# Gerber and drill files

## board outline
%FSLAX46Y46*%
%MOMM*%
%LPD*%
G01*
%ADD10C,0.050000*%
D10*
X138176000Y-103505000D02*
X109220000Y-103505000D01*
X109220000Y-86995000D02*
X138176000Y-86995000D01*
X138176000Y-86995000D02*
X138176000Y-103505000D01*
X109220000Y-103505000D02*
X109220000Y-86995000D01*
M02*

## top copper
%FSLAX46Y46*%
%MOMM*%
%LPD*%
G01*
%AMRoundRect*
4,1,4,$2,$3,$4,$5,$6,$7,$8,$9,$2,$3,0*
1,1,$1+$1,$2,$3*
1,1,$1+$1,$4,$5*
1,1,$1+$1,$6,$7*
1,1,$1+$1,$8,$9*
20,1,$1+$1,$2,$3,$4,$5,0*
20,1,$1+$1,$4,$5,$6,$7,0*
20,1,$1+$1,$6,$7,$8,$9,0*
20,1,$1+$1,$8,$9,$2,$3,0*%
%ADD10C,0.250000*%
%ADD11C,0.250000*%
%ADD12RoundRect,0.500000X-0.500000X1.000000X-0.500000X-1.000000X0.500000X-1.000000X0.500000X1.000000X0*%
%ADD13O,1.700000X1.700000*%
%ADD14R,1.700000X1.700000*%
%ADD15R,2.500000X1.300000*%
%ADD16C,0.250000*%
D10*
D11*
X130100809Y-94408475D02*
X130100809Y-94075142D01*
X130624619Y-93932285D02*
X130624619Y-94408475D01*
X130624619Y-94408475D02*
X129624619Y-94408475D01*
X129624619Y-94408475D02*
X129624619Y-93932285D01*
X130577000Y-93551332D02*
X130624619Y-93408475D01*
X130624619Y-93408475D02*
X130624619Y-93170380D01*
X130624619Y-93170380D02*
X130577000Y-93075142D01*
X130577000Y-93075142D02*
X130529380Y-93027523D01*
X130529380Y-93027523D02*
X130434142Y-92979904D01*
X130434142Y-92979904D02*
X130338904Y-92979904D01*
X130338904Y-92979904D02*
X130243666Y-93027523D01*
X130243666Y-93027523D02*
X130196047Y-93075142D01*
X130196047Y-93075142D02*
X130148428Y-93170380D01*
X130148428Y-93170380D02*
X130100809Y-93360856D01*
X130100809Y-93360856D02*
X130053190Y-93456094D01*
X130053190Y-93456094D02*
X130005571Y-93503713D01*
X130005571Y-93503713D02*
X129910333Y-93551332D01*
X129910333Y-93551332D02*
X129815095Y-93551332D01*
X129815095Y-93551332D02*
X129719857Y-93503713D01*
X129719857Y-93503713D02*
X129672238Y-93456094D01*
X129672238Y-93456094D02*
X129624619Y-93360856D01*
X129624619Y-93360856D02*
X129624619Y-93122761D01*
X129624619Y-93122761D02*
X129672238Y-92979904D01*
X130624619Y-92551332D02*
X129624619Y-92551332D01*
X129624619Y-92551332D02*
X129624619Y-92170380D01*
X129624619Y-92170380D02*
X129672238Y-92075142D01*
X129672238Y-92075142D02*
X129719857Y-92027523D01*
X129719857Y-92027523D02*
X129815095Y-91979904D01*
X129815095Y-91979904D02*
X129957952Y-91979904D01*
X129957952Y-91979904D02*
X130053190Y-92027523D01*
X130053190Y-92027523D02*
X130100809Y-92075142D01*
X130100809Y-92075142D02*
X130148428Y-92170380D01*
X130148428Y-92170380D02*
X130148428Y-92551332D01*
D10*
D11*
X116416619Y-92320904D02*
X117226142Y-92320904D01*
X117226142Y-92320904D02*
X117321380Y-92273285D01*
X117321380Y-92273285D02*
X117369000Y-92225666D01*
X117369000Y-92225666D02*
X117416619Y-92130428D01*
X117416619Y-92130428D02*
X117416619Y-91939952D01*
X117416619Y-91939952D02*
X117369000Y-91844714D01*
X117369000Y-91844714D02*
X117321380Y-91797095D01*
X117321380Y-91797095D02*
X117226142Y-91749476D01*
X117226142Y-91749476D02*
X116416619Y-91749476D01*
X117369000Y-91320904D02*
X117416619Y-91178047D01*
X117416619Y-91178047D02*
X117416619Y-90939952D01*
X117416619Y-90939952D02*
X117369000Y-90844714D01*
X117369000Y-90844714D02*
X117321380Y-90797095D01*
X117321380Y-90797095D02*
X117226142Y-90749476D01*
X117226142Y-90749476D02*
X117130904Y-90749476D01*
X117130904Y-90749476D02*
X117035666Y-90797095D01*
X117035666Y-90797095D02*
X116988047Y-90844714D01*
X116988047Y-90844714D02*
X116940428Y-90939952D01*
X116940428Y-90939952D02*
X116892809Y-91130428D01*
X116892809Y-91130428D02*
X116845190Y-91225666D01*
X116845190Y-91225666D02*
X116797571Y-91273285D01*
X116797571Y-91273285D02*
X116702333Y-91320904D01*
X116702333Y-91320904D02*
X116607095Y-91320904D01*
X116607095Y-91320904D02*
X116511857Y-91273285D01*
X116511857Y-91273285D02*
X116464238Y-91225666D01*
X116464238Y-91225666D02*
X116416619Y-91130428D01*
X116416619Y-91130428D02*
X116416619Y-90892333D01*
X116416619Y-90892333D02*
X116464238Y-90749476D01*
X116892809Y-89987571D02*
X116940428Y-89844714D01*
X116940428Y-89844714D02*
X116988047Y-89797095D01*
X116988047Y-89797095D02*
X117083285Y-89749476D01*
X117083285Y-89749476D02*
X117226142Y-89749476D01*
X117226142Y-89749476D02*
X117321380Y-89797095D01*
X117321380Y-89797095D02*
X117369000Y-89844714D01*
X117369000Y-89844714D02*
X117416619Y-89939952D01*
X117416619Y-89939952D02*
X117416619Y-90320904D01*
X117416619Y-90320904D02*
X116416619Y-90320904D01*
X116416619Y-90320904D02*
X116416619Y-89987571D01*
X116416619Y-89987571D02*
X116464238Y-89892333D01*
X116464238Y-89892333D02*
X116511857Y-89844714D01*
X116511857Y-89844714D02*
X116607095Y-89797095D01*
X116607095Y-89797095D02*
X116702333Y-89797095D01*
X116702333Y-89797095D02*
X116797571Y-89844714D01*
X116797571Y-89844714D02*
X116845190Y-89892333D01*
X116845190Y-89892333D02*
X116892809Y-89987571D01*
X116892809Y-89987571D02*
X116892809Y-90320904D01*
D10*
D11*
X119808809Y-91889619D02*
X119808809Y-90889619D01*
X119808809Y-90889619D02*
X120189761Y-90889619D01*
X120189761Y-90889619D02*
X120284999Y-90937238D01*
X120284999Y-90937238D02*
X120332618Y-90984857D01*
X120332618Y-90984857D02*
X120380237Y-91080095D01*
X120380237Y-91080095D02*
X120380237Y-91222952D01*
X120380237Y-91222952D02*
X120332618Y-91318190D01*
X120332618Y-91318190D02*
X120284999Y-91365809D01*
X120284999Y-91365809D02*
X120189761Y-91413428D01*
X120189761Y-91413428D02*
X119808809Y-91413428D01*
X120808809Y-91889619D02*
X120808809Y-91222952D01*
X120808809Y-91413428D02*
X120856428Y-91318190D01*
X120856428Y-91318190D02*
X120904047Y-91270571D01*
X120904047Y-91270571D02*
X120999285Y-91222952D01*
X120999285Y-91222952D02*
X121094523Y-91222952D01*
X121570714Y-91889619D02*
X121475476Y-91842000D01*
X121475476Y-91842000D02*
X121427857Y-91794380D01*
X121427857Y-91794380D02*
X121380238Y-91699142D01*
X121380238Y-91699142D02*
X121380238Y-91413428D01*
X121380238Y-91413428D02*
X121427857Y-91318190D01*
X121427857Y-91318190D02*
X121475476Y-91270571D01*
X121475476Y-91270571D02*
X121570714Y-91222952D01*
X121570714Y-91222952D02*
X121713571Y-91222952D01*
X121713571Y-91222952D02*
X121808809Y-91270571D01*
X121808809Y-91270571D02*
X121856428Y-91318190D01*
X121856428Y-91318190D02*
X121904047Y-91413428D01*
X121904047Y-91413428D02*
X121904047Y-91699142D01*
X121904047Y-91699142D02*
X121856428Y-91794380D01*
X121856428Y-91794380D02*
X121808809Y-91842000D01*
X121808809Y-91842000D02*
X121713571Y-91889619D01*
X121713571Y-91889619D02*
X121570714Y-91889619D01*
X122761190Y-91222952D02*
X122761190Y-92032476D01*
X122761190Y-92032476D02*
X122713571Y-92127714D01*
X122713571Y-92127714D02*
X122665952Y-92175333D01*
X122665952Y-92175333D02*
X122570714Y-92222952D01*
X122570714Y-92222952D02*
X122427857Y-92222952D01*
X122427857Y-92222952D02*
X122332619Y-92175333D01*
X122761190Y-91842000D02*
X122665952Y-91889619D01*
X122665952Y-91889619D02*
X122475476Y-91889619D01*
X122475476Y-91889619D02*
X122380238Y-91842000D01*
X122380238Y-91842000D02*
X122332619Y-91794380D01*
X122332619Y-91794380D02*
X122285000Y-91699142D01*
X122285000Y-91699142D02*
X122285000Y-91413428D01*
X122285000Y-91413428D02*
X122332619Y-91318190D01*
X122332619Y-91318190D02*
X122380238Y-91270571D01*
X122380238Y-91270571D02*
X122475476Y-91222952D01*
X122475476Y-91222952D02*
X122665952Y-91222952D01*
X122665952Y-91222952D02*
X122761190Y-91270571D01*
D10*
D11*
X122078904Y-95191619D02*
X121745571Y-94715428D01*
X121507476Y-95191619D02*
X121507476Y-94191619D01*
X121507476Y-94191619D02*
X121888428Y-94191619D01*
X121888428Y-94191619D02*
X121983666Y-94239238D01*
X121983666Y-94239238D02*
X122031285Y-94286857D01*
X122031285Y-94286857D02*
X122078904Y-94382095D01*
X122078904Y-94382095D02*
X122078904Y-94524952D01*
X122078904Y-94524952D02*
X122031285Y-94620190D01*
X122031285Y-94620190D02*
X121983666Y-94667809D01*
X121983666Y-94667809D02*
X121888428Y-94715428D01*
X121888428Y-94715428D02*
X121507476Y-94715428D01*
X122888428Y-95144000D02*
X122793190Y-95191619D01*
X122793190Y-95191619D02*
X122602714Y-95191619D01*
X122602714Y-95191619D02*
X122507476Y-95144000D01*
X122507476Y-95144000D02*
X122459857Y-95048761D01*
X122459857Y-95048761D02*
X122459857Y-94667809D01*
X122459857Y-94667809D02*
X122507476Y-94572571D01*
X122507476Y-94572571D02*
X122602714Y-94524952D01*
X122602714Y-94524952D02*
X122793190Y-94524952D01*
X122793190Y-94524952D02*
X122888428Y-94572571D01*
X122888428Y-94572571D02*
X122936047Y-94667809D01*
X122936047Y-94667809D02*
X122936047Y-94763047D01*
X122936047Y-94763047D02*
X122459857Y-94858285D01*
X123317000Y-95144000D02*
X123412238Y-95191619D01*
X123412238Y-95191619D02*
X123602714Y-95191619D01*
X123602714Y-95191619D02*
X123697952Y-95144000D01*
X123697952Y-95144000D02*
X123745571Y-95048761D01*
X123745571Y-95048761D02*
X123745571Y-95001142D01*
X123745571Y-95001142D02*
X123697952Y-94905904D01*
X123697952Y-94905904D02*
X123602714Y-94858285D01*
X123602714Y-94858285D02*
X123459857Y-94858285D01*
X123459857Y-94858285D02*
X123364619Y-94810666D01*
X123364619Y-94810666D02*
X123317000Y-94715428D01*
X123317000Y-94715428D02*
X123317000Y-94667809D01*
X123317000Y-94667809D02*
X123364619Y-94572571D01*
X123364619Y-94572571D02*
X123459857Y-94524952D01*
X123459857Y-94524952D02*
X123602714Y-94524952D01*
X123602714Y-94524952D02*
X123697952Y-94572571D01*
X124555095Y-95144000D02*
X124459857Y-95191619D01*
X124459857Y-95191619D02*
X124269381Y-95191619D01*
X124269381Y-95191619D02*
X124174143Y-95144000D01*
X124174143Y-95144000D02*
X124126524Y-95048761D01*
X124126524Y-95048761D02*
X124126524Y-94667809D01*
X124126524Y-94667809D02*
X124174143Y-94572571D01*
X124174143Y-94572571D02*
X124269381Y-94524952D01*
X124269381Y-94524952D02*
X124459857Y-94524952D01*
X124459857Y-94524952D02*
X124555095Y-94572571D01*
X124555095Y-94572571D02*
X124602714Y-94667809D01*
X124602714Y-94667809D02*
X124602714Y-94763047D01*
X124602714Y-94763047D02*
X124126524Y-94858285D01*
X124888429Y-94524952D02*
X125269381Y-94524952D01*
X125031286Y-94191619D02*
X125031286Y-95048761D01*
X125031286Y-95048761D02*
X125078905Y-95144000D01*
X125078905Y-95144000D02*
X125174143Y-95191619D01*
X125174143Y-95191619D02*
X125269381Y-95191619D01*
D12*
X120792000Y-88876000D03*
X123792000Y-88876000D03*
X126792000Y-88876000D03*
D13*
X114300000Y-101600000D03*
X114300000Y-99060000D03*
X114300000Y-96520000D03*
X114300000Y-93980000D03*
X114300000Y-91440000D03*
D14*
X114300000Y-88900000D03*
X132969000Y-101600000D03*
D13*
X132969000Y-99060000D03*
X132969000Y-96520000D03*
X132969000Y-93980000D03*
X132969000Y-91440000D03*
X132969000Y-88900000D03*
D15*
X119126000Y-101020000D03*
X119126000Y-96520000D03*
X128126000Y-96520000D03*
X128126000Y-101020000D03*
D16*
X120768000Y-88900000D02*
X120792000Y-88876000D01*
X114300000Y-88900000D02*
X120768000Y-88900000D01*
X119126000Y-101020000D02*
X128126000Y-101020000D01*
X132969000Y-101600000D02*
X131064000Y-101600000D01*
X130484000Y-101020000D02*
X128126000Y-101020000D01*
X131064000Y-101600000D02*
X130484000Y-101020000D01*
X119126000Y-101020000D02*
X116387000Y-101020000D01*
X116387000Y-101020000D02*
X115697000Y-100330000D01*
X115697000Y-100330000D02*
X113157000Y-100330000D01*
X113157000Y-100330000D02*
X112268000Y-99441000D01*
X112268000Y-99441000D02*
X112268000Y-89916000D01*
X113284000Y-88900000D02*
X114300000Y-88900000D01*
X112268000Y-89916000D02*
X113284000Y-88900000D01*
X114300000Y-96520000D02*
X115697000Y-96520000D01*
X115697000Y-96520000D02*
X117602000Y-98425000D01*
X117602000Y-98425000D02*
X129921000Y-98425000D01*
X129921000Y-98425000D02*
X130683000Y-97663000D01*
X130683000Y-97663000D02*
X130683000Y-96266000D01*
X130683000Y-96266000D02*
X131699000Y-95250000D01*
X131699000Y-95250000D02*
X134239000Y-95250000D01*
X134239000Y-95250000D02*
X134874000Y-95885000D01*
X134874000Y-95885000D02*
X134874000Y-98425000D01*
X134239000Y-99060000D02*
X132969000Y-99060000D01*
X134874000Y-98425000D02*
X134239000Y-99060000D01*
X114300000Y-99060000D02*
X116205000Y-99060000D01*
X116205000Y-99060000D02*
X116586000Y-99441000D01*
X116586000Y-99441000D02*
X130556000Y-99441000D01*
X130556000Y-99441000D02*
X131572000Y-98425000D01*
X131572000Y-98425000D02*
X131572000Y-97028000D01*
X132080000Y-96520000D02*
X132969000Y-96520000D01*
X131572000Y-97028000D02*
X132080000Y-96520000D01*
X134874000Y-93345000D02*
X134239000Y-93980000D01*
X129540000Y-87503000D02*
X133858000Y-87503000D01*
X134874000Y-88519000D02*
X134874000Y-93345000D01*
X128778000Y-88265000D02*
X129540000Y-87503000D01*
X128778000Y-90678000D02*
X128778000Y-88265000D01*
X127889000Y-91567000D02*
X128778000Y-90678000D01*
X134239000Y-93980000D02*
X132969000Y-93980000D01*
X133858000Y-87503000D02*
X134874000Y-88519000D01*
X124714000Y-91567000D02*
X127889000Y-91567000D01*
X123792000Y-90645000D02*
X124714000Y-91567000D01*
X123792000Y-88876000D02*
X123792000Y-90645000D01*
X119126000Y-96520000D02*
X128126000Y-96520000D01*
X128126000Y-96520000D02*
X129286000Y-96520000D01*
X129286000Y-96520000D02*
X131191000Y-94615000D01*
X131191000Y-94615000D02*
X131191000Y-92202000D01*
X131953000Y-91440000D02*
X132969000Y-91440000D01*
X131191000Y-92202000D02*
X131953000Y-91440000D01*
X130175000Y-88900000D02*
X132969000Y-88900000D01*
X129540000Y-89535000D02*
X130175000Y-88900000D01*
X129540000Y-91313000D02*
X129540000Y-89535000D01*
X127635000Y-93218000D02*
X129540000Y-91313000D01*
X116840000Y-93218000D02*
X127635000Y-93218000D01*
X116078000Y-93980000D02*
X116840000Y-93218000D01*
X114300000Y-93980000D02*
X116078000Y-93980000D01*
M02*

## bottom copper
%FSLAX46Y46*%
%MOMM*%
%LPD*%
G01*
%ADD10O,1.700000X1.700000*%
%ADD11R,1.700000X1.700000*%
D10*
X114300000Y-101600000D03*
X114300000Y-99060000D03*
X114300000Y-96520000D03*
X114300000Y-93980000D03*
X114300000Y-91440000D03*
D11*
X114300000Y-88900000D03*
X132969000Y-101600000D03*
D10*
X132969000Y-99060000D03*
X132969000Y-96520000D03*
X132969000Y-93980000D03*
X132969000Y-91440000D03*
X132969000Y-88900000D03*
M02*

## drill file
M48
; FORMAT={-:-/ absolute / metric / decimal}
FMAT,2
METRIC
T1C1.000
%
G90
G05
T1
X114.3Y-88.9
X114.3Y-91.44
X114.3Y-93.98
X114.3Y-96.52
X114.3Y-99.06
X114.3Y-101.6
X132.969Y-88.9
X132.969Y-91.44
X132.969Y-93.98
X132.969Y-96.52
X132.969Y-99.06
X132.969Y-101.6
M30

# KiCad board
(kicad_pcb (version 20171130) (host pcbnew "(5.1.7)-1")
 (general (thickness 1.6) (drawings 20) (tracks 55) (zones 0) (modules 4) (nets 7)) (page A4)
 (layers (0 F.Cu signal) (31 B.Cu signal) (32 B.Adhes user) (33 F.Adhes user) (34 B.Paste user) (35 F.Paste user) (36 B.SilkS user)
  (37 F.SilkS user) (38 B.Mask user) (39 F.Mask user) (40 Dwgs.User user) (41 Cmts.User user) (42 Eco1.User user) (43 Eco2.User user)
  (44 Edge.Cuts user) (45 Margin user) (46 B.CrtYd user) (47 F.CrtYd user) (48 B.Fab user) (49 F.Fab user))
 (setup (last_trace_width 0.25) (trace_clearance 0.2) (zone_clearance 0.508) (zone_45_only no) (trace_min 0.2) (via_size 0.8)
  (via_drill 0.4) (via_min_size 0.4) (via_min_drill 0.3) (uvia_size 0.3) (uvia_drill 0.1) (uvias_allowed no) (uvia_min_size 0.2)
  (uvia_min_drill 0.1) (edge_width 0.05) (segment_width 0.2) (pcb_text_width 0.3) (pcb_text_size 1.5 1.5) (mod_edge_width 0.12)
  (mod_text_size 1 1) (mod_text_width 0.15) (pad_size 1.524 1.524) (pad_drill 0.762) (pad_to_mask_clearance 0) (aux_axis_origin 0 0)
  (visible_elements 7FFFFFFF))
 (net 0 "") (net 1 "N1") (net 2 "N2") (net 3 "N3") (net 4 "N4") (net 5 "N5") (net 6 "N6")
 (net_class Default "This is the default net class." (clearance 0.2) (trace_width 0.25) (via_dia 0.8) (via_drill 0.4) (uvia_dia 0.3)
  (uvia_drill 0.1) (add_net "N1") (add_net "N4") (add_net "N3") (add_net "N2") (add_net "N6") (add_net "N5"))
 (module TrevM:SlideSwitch (layer F.Cu) (at 113.792 87.376 270)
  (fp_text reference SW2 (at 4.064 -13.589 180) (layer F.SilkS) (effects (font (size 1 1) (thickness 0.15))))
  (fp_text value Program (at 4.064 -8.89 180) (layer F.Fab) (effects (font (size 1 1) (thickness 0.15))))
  (pad 1 smd roundrect (at 1.5 -7 270) (size 3 2) (layers F.Cu F.Paste F.Mask) (roundrect_rratio 0.25) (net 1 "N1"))
  (pad 2 smd roundrect (at 1.5 -10 270) (size 3 2) (layers F.Cu F.Paste F.Mask) (roundrect_rratio 0.25) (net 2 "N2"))
  (pad 3 smd roundrect (at 1.5 -13 270) (size 3 2) (layers F.Cu F.Paste F.Mask) (roundrect_rratio 0.25)))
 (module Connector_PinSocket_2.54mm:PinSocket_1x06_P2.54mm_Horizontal (layer F.Cu) (at 114.3 88.9)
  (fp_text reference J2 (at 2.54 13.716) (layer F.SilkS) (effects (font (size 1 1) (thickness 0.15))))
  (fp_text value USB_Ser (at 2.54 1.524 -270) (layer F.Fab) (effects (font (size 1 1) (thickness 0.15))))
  (pad 6 thru_hole oval (at 0 12.7) (size 1.7 1.7) (drill 1) (layers *.Cu *.Mask))
  (pad 5 thru_hole oval (at 0 10.16) (size 1.7 1.7) (drill 1) (layers *.Cu *.Mask) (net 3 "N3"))
  (pad 4 thru_hole oval (at 0 7.62) (size 1.7 1.7) (drill 1) (layers *.Cu *.Mask) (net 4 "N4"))
  (pad 3 thru_hole oval (at 0 5.08) (size 1.7 1.7) (drill 1) (layers *.Cu *.Mask) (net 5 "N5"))
  (pad 2 thru_hole oval (at 0 2.54) (size 1.7 1.7) (drill 1) (layers *.Cu *.Mask))
  (pad 1 thru_hole rect (at 0 0) (size 1.7 1.7) (drill 1) (layers *.Cu *.Mask) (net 1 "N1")))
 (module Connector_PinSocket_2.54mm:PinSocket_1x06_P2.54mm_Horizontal (layer F.Cu) (at 132.969 101.6 180)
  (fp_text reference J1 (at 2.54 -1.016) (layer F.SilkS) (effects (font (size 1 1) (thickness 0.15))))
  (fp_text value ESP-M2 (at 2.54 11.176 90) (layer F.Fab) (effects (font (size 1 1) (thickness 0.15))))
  (pad 1 thru_hole rect (at 0 0 180) (size 1.7 1.7) (drill 1) (layers *.Cu *.Mask) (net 1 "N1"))
  (pad 2 thru_hole oval (at 0 2.54 180) (size 1.7 1.7) (drill 1) (layers *.Cu *.Mask) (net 4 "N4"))
  (pad 3 thru_hole oval (at 0 5.08 180) (size 1.7 1.7) (drill 1) (layers *.Cu *.Mask) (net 3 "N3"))
  (pad 4 thru_hole oval (at 0 7.62 180) (size 1.7 1.7) (drill 1) (layers *.Cu *.Mask) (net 2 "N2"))
  (pad 5 thru_hole oval (at 0 10.16 180) (size 1.7 1.7) (drill 1) (layers *.Cu *.Mask) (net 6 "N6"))
  (pad 6 thru_hole oval (at 0 12.7 180) (size 1.7 1.7) (drill 1) (layers *.Cu *.Mask) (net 5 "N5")))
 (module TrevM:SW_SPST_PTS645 (layer F.Cu) (at 123.626 98.77)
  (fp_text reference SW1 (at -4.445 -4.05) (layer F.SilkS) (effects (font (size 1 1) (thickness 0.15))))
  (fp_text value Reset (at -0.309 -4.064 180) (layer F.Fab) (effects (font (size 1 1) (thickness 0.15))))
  (pad 2 smd rect (at -4.5 2.25) (size 2.5 1.3) (layers F.Cu F.Paste F.Mask) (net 1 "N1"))
  (pad 1 smd rect (at -4.5 -2.25) (size 2.5 1.3) (layers F.Cu F.Paste F.Mask) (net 6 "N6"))
  (pad 1 smd rect (at 4.5 -2.25) (size 2.5 1.3) (layers F.Cu F.Paste F.Mask) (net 6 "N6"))
  (pad 2 smd rect (at 4.5 2.25) (size 2.5 1.3) (layers F.Cu F.Paste F.Mask) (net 1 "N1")))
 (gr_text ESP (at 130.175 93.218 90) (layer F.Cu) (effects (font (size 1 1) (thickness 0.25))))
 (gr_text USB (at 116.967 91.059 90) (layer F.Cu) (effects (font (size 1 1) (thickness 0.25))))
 (gr_line (start 138.176 103.505) (end 109.22 103.505) (layer Edge.Cuts) (width 0.05))
 (gr_line (start 109.22 86.995) (end 138.176 86.995) (layer Edge.Cuts) (width 0.05))
 (gr_line (start 138.176 86.995) (end 138.176 103.505) (layer Edge.Cuts) (width 0.05))
 (gr_line (start 109.22 103.505) (end 109.22 86.995) (layer Edge.Cuts) (width 0.05))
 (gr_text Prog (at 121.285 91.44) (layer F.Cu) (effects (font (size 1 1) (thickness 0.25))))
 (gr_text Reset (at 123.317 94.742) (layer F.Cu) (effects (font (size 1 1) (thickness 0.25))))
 (segment (start 120.768 88.9) (end 120.792 88.876) (width 0.25) (layer F.Cu) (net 1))
 (segment (start 114.3 88.9) (end 120.768 88.9) (width 0.25) (layer F.Cu) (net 1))
 (segment (start 119.126 101.02) (end 128.126 101.02) (width 0.25) (layer F.Cu) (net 1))
 (segment (start 132.969 101.6) (end 131.064 101.6) (width 0.25) (layer F.Cu) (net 1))
 (segment (start 130.484 101.02) (end 128.126 101.02) (width 0.25) (layer F.Cu) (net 1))
 (segment (start 131.064 101.6) (end 130.484 101.02) (width 0.25) (layer F.Cu) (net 1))
 (segment (start 119.126 101.02) (end 116.387 101.02) (width 0.25) (layer F.Cu) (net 1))
 (segment (start 116.387 101.02) (end 115.697 100.33) (width 0.25) (layer F.Cu) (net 1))
 (segment (start 115.697 100.33) (end 113.157 100.33) (width 0.25) (layer F.Cu) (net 1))
 (segment (start 113.157 100.33) (end 112.268 99.441) (width 0.25) (layer F.Cu) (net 1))
 (segment (start 112.268 99.441) (end 112.268 89.916) (width 0.25) (layer F.Cu) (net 1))
 (segment (start 113.284 88.9) (end 114.3 88.9) (width 0.25) (layer F.Cu) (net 1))
 (segment (start 112.268 89.916) (end 113.284 88.9) (width 0.25) (layer F.Cu) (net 1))
 (segment (start 114.3 96.52) (end 115.697 96.52) (width 0.25) (layer F.Cu) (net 4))
 (segment (start 115.697 96.52) (end 117.602 98.425) (width 0.25) (layer F.Cu) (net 4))
 (segment (start 117.602 98.425) (end 129.921 98.425) (width 0.25) (layer F.Cu) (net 4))
 (segment (start 129.921 98.425) (end 130.683 97.663) (width 0.25) (layer F.Cu) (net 4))
 (segment (start 130.683 97.663) (end 130.683 96.266) (width 0.25) (layer F.Cu) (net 4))
 (segment (start 130.683 96.266) (end 131.699 95.25) (width 0.25) (layer F.Cu) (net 4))
 (segment (start 131.699 95.25) (end 134.239 95.25) (width 0.25) (layer F.Cu) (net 4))
 (segment (start 134.239 95.25) (end 134.874 95.885) (width 0.25) (layer F.Cu) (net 4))
 (segment (start 134.874 95.885) (end 134.874 98.425) (width 0.25) (layer F.Cu) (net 4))
 (segment (start 134.239 99.06) (end 132.969 99.06) (width 0.25) (layer F.Cu) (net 4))
 (segment (start 134.874 98.425) (end 134.239 99.06) (width 0.25) (layer F.Cu) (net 4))
 (segment (start 114.3 99.06) (end 116.205 99.06) (width 0.25) (layer F.Cu) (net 3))
 (segment (start 116.205 99.06) (end 116.586 99.441) (width 0.25) (layer F.Cu) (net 3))
 (segment (start 116.586 99.441) (end 130.556 99.441) (width 0.25) (layer F.Cu) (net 3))
 (segment (start 130.556 99.441) (end 131.572 98.425) (width 0.25) (layer F.Cu) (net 3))
 (segment (start 131.572 98.425) (end 131.572 97.028) (width 0.25) (layer F.Cu) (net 3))
 (segment (start 132.08 96.52) (end 132.969 96.52) (width 0.25) (layer F.Cu) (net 3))
 (segment (start 131.572 97.028) (end 132.08 96.52) (width 0.25) (layer F.Cu) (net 3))
 (segment (start 134.874 93.345) (end 134.239 93.98) (width 0.25) (layer F.Cu) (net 2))
 (segment (start 129.54 87.503) (end 133.858 87.503) (width 0.25) (layer F.Cu) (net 2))
 (segment (start 134.874 88.519) (end 134.874 93.345) (width 0.25) (layer F.Cu) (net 2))
 (segment (start 128.778 88.265) (end 129.54 87.503) (width 0.25) (layer F.Cu) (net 2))
 (segment (start 128.778 90.678) (end 128.778 88.265) (width 0.25) (layer F.Cu) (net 2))
 (segment (start 127.889 91.567) (end 128.778 90.678) (width 0.25) (layer F.Cu) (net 2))
 (segment (start 134.239 93.98) (end 132.969 93.98) (width 0.25) (layer F.Cu) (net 2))
 (segment (start 133.858 87.503) (end 134.874 88.519) (width 0.25) (layer F.Cu) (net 2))
 (segment (start 124.714 91.567) (end 127.889 91.567) (width 0.25) (layer F.Cu) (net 2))
 (segment (start 123.792 90.645) (end 124.714 91.567) (width 0.25) (layer F.Cu) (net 2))
 (segment (start 123.792 88.876) (end 123.792 90.645) (width 0.25) (layer F.Cu) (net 2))
 (segment (start 119.126 96.52) (end 128.126 96.52) (width 0.25) (layer F.Cu) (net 6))
 (segment (start 128.126 96.52) (end 129.286 96.52) (width 0.25) (layer F.Cu) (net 6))
 (segment (start 129.286 96.52) (end 131.191 94.615) (width 0.25) (layer F.Cu) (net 6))
 (segment (start 131.191 94.615) (end 131.191 92.202) (width 0.25) (layer F.Cu) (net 6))
 (segment (start 131.953 91.44) (end 132.969 91.44) (width 0.25) (layer F.Cu) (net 6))
 (segment (start 131.191 92.202) (end 131.953 91.44) (width 0.25) (layer F.Cu) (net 6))
 (segment (start 130.175 88.9) (end 132.969 88.9) (width 0.25) (layer F.Cu) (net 5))
 (segment (start 129.54 89.535) (end 130.175 88.9) (width 0.25) (layer F.Cu) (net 5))
 (segment (start 129.54 91.313) (end 129.54 89.535) (width 0.25) (layer F.Cu) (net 5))
 (segment (start 127.635 93.218) (end 129.54 91.313) (width 0.25) (layer F.Cu) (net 5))
 (segment (start 116.84 93.218) (end 127.635 93.218) (width 0.25) (layer F.Cu) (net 5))
 (segment (start 116.078 93.98) (end 116.84 93.218) (width 0.25) (layer F.Cu) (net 5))
 (segment (start 114.3 93.98) (end 116.078 93.98) (width 0.25) (layer F.Cu) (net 5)))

